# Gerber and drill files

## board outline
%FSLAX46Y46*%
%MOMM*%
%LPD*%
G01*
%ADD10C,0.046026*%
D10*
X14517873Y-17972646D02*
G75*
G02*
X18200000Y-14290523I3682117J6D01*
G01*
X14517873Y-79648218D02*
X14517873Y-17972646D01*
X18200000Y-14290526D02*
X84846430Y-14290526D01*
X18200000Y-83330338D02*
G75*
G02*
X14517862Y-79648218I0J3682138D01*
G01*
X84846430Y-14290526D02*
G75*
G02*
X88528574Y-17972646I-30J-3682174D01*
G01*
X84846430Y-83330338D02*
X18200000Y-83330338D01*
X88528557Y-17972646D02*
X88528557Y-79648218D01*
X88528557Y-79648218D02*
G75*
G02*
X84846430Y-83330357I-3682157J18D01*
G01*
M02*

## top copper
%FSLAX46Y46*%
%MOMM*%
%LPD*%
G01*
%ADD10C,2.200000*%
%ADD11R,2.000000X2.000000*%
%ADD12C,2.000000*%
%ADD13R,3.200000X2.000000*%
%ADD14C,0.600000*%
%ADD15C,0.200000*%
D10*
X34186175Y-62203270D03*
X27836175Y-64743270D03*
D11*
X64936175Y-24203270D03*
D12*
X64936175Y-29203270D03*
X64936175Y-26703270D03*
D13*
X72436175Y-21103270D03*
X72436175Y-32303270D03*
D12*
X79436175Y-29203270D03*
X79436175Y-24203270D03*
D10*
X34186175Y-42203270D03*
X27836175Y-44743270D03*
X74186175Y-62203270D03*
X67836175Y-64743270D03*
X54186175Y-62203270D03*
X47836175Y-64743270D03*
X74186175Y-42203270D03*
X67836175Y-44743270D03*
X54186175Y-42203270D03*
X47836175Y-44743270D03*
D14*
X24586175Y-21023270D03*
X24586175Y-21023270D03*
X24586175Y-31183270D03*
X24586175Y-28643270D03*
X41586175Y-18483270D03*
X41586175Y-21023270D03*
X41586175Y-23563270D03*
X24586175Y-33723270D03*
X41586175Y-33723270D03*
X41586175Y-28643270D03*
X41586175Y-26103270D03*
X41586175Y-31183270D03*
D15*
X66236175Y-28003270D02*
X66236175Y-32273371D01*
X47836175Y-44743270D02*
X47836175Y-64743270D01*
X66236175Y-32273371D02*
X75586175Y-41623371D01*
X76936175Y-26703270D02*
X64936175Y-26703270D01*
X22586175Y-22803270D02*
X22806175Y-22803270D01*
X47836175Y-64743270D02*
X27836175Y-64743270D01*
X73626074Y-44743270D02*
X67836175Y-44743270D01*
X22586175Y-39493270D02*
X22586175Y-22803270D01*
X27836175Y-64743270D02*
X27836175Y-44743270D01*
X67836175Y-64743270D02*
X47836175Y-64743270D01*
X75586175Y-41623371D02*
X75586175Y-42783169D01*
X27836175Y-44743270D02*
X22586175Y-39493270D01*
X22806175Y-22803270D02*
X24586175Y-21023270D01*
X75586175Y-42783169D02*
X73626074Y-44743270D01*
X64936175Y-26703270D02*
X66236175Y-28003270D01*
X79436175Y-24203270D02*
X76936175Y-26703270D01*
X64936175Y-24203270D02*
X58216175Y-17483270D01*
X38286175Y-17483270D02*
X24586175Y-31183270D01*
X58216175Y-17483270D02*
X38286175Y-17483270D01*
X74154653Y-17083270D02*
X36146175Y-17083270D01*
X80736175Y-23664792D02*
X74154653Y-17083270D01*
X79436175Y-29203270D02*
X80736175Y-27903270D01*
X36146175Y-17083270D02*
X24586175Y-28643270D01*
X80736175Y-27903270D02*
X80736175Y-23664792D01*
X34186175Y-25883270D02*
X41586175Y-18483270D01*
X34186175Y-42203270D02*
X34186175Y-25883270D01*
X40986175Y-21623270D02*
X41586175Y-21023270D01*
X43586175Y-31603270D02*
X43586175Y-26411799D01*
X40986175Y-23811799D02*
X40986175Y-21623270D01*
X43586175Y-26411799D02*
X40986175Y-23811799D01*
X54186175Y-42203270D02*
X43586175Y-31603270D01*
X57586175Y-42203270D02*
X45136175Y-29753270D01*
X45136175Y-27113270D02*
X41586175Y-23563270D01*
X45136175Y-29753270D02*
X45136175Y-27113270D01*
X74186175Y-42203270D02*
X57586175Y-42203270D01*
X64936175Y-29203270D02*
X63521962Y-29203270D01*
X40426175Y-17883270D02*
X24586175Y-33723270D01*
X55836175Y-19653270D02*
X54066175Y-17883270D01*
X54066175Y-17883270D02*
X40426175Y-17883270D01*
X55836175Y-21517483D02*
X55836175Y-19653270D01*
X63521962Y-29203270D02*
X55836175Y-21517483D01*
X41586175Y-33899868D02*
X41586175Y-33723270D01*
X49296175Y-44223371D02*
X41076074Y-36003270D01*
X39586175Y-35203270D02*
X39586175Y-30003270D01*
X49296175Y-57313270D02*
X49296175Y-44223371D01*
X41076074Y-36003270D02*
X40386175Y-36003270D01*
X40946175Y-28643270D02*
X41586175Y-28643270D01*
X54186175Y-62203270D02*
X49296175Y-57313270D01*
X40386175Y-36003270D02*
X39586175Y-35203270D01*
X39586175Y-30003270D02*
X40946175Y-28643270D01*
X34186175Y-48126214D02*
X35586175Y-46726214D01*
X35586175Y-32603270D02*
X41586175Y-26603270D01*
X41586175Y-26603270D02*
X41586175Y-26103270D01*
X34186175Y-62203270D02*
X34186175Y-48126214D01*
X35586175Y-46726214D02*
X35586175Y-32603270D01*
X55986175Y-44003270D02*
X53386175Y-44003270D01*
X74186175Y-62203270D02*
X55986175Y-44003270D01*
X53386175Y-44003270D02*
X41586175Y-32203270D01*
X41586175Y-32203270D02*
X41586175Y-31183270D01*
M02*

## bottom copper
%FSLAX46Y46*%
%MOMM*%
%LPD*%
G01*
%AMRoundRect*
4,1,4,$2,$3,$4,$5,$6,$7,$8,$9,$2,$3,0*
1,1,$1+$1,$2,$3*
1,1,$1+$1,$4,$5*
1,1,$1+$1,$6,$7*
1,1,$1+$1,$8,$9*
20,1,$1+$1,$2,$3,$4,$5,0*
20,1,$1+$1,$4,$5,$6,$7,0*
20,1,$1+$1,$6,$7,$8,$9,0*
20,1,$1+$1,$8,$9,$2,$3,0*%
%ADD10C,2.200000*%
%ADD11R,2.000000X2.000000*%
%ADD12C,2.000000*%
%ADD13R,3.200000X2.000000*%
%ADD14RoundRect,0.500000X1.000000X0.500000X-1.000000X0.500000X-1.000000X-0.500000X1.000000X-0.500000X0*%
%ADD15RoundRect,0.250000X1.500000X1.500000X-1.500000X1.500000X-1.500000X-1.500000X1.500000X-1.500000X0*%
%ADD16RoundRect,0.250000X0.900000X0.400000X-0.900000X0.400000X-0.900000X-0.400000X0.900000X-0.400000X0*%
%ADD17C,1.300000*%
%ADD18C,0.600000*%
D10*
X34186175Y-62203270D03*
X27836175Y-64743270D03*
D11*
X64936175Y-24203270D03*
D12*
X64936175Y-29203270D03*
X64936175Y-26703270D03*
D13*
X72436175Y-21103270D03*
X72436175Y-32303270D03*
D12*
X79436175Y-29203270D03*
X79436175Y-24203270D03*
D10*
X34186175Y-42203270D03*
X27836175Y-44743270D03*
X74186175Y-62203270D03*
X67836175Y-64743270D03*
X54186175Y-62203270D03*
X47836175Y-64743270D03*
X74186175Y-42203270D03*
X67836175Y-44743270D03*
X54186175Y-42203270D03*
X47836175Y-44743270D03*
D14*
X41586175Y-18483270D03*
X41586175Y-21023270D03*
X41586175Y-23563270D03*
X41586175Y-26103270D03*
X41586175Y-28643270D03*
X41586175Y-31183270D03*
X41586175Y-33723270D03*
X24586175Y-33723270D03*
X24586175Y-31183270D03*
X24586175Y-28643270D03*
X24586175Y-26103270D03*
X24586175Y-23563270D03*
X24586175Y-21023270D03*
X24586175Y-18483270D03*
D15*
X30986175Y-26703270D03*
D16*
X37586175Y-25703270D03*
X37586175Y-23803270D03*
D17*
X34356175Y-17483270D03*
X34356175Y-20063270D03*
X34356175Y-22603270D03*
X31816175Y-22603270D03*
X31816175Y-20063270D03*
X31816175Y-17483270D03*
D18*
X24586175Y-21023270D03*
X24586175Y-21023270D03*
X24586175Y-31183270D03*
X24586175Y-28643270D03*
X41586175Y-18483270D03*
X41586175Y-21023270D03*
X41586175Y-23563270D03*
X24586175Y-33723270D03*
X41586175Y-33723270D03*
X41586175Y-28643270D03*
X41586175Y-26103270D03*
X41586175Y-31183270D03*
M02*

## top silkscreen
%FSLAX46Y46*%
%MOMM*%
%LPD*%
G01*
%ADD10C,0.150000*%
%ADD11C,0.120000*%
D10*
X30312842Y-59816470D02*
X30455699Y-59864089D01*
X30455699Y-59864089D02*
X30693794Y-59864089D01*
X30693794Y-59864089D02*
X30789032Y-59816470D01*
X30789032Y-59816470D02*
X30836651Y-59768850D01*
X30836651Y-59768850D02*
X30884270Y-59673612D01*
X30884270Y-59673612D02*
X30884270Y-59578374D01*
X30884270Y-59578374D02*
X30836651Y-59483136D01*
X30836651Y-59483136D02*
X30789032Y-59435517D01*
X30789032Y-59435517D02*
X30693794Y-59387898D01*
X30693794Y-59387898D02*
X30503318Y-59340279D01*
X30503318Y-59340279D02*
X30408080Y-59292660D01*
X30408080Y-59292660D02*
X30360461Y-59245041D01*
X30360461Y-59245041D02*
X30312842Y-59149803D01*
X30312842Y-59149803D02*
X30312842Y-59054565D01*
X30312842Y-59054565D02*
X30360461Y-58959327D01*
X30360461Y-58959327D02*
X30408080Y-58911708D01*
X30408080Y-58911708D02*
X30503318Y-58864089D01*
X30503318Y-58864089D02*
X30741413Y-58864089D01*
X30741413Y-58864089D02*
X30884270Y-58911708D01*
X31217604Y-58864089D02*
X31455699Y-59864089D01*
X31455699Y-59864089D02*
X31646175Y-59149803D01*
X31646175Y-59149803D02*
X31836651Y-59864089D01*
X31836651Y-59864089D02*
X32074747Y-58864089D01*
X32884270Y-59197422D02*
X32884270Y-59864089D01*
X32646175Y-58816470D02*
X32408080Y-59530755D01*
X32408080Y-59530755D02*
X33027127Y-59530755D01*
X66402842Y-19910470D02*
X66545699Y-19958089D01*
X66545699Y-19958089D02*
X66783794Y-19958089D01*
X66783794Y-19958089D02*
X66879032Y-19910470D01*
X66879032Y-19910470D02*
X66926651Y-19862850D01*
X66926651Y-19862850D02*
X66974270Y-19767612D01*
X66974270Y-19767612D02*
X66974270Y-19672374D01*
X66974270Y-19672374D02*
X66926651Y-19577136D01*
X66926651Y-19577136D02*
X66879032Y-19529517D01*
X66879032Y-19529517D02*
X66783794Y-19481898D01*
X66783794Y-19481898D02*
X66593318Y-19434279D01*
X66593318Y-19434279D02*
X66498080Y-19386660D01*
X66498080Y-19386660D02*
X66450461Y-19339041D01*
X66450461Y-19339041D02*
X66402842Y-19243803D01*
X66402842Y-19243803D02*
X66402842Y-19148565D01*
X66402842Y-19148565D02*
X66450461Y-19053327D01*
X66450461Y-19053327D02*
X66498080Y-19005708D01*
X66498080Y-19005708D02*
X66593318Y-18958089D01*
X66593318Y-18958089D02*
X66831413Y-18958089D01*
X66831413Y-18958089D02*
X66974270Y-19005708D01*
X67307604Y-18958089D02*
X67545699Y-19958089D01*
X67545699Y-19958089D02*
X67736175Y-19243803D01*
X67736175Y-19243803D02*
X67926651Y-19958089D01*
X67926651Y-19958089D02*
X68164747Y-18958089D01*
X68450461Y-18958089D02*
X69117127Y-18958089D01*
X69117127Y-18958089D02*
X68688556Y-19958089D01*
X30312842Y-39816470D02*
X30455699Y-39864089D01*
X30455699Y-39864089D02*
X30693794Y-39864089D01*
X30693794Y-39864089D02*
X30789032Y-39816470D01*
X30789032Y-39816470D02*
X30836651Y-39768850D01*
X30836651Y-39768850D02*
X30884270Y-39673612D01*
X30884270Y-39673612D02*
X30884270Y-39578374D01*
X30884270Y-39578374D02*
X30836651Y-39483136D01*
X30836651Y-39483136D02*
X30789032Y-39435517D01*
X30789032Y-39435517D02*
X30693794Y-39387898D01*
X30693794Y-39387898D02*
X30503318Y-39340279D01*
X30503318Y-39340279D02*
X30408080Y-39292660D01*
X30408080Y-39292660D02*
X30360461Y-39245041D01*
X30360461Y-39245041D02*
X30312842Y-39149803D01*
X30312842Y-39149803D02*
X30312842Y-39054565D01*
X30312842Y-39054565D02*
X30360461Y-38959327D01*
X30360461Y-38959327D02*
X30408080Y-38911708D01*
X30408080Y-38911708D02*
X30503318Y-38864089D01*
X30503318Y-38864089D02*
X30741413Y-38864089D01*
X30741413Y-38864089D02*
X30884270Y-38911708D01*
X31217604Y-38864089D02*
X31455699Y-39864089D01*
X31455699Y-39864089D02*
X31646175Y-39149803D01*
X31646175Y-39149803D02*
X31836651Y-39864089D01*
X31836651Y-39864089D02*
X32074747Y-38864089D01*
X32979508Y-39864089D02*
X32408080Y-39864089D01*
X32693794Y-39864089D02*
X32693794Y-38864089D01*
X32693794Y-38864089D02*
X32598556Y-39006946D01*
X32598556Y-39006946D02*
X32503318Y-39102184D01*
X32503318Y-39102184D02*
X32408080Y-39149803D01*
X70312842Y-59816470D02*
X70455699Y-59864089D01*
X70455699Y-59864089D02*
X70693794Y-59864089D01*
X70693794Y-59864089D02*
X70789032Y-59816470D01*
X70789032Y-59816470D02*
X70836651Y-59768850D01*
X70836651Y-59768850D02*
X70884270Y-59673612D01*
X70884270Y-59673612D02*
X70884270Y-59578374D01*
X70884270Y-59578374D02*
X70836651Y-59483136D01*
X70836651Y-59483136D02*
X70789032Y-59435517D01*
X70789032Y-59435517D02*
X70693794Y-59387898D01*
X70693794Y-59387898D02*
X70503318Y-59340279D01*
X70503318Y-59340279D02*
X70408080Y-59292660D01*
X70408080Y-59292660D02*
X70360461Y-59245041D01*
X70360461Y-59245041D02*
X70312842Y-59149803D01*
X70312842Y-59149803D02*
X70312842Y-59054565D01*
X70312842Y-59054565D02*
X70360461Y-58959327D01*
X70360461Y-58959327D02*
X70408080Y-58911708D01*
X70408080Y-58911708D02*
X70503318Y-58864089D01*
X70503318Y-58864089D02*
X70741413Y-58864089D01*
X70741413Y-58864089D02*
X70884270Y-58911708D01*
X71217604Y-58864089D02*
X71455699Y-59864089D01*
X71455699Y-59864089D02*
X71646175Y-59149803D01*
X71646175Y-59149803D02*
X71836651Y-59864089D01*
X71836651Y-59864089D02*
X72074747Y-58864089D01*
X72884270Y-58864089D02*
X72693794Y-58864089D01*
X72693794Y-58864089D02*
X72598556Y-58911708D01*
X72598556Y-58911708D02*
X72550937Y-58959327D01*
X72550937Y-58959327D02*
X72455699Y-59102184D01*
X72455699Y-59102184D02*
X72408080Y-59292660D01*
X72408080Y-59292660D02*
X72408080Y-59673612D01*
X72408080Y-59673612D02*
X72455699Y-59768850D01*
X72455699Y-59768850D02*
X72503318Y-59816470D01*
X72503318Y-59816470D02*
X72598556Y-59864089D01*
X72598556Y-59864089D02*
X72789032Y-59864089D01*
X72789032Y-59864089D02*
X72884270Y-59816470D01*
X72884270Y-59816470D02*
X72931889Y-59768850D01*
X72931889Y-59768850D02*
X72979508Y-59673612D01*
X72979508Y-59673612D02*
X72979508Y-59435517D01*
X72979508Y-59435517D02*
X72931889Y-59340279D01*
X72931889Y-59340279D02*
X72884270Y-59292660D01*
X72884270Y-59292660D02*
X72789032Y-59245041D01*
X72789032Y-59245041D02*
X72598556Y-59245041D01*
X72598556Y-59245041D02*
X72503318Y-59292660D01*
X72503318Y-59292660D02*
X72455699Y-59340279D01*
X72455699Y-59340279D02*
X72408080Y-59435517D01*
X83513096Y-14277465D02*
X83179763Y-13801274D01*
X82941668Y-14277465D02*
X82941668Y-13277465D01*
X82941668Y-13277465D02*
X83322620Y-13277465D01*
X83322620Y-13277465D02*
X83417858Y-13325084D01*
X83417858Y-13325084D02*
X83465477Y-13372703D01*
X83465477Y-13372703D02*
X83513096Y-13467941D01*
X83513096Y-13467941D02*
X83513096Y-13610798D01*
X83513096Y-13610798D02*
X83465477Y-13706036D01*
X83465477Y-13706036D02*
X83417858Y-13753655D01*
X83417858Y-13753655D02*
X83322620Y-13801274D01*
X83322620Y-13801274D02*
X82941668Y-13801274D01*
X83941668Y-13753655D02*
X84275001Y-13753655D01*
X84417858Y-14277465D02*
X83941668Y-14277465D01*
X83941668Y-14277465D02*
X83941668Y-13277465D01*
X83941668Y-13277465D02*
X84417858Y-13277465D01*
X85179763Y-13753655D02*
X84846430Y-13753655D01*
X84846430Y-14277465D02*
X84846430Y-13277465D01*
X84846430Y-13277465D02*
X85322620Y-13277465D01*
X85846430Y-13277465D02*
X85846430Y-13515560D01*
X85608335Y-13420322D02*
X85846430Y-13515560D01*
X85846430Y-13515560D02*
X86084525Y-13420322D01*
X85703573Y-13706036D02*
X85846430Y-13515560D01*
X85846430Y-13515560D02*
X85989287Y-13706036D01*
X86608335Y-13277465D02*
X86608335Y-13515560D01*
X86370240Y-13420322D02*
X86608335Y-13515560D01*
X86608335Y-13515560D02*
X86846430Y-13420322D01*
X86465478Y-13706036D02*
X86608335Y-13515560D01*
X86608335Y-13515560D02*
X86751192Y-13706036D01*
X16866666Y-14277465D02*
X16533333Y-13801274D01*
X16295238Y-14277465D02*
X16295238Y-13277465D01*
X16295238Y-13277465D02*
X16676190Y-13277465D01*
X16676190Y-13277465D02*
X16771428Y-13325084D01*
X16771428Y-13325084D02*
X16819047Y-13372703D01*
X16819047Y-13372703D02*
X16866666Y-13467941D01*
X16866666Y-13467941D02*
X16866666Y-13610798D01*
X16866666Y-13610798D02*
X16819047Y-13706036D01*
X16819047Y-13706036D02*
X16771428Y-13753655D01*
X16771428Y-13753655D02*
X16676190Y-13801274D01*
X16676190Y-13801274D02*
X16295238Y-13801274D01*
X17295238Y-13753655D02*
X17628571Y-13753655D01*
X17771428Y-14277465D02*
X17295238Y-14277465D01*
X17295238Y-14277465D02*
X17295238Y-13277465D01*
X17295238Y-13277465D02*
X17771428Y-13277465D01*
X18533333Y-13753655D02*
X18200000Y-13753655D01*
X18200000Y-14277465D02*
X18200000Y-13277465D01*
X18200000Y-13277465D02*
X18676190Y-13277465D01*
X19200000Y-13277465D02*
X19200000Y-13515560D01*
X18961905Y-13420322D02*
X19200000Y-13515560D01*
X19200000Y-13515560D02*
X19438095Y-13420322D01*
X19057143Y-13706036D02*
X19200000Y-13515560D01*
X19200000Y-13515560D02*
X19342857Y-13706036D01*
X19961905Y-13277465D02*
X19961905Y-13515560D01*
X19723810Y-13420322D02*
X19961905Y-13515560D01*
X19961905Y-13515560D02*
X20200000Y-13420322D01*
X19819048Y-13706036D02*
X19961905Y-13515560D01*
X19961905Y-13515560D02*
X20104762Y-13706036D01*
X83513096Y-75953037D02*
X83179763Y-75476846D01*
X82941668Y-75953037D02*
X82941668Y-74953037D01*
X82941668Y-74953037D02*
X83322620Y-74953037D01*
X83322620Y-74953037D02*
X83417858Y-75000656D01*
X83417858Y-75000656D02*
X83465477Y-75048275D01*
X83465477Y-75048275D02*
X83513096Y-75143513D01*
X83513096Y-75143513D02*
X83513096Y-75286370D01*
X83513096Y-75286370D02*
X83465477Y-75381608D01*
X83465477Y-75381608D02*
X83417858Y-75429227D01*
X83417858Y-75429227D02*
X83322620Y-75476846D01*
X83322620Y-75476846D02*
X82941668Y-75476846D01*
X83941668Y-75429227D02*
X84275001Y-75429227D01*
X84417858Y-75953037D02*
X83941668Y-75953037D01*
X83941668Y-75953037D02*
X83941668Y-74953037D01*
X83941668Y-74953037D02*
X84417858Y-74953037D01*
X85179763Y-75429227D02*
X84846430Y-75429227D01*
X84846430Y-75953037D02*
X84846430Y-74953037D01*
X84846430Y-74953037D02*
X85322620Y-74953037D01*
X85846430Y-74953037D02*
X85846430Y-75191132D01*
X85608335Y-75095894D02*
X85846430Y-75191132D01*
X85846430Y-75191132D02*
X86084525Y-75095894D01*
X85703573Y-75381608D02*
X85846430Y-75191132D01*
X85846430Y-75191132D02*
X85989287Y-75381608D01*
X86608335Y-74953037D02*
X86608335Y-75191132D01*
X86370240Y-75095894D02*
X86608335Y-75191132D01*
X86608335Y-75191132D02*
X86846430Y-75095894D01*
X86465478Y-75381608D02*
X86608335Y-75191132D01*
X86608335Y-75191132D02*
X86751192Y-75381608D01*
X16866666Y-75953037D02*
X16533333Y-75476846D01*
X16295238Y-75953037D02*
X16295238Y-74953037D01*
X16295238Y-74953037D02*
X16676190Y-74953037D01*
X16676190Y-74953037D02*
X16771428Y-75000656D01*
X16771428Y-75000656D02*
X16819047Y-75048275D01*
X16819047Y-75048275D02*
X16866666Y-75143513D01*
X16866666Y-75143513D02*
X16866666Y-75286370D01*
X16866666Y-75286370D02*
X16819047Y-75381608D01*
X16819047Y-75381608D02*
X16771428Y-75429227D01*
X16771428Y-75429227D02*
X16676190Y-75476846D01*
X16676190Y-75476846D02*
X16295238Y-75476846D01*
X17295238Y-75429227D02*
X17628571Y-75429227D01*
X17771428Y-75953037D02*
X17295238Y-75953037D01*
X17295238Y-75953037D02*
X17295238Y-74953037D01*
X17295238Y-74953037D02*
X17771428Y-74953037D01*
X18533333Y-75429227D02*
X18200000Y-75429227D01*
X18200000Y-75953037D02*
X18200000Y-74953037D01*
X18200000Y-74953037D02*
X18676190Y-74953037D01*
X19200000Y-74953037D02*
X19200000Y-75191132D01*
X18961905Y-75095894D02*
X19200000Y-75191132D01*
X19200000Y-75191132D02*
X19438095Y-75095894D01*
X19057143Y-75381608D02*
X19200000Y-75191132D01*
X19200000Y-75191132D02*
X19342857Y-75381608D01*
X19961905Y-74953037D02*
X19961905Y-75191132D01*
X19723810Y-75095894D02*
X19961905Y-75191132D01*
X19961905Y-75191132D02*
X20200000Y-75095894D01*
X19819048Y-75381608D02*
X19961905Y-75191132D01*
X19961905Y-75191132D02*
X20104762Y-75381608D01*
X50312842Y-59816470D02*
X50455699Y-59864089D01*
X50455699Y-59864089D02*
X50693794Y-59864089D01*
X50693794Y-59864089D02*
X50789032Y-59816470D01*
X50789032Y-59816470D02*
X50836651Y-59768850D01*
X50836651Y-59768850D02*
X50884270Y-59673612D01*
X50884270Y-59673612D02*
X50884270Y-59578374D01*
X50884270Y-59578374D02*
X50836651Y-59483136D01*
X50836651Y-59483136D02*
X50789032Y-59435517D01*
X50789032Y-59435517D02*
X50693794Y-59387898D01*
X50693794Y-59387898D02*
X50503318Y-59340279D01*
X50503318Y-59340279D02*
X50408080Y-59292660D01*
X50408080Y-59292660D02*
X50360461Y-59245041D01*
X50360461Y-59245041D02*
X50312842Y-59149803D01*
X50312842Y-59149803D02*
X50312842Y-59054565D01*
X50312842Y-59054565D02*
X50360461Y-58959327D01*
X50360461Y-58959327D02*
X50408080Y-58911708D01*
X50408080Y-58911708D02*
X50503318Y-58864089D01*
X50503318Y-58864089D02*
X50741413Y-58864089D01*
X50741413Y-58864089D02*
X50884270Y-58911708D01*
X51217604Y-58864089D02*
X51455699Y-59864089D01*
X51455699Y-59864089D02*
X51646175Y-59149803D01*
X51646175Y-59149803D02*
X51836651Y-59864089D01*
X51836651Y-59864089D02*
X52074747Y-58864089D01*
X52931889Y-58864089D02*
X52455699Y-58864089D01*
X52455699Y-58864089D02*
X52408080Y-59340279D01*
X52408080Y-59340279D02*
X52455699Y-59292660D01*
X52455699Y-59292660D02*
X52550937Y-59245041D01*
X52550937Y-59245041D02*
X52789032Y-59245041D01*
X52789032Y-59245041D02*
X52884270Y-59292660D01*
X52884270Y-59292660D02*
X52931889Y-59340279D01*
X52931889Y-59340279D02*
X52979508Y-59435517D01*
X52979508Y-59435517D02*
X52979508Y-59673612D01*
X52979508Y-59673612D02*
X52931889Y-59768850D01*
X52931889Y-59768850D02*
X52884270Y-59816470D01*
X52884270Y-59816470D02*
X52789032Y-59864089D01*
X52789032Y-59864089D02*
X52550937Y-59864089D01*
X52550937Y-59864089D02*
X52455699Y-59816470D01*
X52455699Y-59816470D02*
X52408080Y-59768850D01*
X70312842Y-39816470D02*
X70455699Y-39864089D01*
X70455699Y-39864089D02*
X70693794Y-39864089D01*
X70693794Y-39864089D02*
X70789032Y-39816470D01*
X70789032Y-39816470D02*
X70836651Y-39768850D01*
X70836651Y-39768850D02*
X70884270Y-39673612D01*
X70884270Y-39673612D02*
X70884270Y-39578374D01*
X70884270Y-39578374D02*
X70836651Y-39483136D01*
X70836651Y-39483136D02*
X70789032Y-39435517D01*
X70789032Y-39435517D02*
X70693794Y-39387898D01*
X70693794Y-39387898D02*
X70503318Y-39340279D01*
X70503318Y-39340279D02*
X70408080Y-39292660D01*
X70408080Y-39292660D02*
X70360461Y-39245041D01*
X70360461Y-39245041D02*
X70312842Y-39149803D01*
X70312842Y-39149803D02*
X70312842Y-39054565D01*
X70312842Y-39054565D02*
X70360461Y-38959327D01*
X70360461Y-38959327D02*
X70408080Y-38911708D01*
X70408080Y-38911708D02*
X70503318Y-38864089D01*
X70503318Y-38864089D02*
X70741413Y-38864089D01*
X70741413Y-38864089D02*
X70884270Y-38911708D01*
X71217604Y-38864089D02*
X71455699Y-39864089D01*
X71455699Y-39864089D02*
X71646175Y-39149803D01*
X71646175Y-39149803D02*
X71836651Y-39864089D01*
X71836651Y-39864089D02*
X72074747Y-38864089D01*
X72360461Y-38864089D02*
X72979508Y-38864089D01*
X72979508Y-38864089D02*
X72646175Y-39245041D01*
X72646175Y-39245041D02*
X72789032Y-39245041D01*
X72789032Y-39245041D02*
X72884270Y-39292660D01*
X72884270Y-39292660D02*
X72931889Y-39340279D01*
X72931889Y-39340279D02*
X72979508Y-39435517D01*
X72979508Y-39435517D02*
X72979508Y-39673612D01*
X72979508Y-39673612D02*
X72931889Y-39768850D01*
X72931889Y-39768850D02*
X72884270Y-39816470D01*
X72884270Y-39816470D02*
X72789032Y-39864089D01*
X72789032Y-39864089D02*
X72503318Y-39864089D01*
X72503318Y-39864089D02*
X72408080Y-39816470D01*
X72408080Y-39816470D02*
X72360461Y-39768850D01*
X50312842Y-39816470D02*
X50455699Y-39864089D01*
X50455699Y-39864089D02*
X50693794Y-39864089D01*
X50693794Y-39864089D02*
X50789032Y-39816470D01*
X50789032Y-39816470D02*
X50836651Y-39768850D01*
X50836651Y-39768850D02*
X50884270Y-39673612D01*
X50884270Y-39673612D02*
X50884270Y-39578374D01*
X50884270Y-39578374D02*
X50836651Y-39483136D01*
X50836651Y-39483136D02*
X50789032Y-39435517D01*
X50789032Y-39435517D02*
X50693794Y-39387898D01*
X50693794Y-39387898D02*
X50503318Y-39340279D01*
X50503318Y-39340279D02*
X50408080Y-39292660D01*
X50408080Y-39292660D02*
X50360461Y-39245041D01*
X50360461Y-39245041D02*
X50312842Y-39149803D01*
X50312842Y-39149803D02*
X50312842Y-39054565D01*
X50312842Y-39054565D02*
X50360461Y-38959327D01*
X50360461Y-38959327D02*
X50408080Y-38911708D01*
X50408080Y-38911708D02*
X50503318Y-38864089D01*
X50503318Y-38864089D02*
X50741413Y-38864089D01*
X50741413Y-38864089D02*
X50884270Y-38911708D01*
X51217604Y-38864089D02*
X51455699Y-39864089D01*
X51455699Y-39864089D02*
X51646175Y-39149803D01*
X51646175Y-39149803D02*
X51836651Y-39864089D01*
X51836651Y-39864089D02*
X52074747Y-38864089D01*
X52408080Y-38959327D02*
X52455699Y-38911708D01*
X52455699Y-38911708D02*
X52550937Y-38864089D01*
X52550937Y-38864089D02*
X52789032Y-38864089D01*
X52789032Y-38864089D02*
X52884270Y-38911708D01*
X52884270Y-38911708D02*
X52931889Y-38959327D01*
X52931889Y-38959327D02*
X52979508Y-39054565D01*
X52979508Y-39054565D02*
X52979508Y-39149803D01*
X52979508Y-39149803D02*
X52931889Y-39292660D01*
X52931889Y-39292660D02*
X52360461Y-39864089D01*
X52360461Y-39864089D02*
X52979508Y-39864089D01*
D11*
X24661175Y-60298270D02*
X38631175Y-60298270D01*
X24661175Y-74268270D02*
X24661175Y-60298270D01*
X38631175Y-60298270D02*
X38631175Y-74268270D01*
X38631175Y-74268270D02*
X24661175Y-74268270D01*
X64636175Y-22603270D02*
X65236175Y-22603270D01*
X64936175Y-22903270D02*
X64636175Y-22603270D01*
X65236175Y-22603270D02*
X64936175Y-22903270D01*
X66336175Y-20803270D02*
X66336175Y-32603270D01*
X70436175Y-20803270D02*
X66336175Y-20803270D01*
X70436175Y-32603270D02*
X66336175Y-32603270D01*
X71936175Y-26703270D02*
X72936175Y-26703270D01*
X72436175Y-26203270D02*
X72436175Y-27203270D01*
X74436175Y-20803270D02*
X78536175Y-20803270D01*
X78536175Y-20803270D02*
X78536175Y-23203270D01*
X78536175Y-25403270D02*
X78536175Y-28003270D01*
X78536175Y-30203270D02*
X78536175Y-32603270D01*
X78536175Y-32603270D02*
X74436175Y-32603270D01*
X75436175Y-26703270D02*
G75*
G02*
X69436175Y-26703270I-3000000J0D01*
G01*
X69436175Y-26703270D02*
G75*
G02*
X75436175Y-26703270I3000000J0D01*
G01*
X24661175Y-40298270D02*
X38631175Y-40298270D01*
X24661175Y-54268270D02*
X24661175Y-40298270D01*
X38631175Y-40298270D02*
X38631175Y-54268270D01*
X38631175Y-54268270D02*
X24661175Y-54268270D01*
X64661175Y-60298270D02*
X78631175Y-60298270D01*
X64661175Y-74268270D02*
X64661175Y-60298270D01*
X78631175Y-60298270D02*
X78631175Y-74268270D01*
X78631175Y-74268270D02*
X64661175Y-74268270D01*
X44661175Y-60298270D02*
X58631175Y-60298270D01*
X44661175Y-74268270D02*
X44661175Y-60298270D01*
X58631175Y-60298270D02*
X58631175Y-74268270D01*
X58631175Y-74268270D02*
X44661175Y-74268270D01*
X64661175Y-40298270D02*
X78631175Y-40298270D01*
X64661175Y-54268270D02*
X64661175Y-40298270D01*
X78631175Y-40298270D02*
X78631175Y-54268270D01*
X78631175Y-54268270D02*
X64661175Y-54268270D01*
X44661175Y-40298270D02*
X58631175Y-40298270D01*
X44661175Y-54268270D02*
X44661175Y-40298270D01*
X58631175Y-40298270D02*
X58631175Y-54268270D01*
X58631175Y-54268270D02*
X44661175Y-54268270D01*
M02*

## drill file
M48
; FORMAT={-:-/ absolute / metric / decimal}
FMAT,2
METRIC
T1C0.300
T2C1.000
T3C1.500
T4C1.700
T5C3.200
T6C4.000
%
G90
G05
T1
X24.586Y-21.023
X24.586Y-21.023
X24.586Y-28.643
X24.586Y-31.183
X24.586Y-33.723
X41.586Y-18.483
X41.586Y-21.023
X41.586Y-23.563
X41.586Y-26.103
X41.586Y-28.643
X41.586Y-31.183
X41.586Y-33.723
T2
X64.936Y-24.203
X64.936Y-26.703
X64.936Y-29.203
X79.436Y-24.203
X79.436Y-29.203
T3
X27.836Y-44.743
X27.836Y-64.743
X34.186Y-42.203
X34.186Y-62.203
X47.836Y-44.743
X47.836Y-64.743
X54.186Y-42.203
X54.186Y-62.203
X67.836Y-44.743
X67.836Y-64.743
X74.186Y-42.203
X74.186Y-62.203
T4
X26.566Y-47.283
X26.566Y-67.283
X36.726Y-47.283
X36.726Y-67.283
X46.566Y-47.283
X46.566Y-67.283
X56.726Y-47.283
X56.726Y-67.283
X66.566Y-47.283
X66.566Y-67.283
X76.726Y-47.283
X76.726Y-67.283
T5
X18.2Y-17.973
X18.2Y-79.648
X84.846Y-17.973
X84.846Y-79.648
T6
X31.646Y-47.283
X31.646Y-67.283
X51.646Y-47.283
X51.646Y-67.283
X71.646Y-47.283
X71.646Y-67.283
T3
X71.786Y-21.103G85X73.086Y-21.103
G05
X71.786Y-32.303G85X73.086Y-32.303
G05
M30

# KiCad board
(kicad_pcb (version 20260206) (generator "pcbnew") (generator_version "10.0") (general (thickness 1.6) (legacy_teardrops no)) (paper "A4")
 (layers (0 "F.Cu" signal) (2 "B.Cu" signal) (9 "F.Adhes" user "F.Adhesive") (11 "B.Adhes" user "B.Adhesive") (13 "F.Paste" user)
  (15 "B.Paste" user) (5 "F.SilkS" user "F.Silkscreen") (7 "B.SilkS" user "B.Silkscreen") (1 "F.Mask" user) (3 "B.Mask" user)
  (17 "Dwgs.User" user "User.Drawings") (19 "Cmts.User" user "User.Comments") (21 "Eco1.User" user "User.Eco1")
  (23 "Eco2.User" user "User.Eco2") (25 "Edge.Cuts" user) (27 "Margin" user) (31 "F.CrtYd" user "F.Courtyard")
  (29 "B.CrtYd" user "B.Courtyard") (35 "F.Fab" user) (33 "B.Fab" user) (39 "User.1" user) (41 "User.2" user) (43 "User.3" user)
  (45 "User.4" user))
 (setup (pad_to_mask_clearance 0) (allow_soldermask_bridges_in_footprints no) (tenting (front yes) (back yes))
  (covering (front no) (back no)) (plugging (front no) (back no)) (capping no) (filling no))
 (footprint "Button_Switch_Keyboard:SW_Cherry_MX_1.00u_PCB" (layer "F.Cu") (at 34.186175 62.20327)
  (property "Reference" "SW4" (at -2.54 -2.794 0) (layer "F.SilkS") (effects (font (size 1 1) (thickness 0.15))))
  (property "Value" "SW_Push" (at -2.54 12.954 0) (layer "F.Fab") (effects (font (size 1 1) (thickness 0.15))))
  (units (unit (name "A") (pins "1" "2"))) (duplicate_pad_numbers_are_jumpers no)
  (fp_line (start -9.525 -1.905) (end 4.445 -1.905) (stroke (width 0.12) (type solid)) (layer "F.SilkS"))
  (fp_line (start -9.525 12.065) (end -9.525 -1.905) (stroke (width 0.12) (type solid)) (layer "F.SilkS"))
  (fp_line (start 4.445 -1.905) (end 4.445 12.065) (stroke (width 0.12) (type solid)) (layer "F.SilkS"))
  (fp_line (start 4.445 12.065) (end -9.525 12.065) (stroke (width 0.12) (type solid)) (layer "F.SilkS"))
  (pad "" np_thru_hole circle (at -7.62 5.08) (size 1.7 1.7) (drill 1.7) (layers "*.Cu" "*.Mask"))
  (pad "" np_thru_hole circle (at -2.54 5.08) (size 4 4) (drill 4) (layers "*.Cu" "*.Mask"))
  (pad "" np_thru_hole circle (at 2.54 5.08) (size 1.7 1.7) (drill 1.7) (layers "*.Cu" "*.Mask"))
  (pad "1" thru_hole circle (at 0 0) (size 2.2 2.2) (drill 1.5) (layers "*.Cu" "*.Mask") (remove_unused_layers no)
   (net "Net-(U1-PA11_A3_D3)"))
  (pad "2" thru_hole circle (at -6.35 2.54) (size 2.2 2.2) (drill 1.5) (layers "*.Cu" "*.Mask") (remove_unused_layers no)
   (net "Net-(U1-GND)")))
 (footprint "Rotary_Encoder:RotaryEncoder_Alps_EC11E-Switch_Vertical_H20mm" (layer "F.Cu") (at 64.936175 24.20327)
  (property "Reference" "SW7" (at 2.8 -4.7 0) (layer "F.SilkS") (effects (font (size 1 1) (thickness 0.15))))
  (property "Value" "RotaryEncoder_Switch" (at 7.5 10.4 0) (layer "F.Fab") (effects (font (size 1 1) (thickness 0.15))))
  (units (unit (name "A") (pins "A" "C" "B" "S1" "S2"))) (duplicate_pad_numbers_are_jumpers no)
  (fp_line (start -0.3 -1.6) (end 0.3 -1.6) (stroke (width 0.12) (type solid)) (layer "F.SilkS"))
  (fp_line (start 0 -1.3) (end -0.3 -1.6) (stroke (width 0.12) (type solid)) (layer "F.SilkS"))
  (fp_line (start 0.3 -1.6) (end 0 -1.3) (stroke (width 0.12) (type solid)) (layer "F.SilkS"))
  (fp_line (start 1.4 -3.4) (end 1.4 8.4) (stroke (width 0.12) (type solid)) (layer "F.SilkS"))
  (fp_line (start 5.5 -3.4) (end 1.4 -3.4) (stroke (width 0.12) (type solid)) (layer "F.SilkS"))
  (fp_line (start 5.5 8.4) (end 1.4 8.4) (stroke (width 0.12) (type solid)) (layer "F.SilkS"))
  (fp_line (start 7 2.5) (end 8 2.5) (stroke (width 0.12) (type solid)) (layer "F.SilkS"))
  (fp_line (start 7.5 2) (end 7.5 3) (stroke (width 0.12) (type solid)) (layer "F.SilkS"))
  (fp_line (start 9.5 -3.4) (end 13.6 -3.4) (stroke (width 0.12) (type solid)) (layer "F.SilkS"))
  (fp_line (start 13.6 -3.4) (end 13.6 -1) (stroke (width 0.12) (type solid)) (layer "F.SilkS"))
  (fp_line (start 13.6 1.2) (end 13.6 3.8) (stroke (width 0.12) (type solid)) (layer "F.SilkS"))
  (fp_line (start 13.6 6) (end 13.6 8.4) (stroke (width 0.12) (type solid)) (layer "F.SilkS"))
  (fp_line (start 13.6 8.4) (end 9.5 8.4) (stroke (width 0.12) (type solid)) (layer "F.SilkS"))
  (fp_circle (center 7.5 2.5) (end 10.5 2.5) (stroke (width 0.12) (type solid)) (fill no) (layer "F.SilkS"))
  (pad "A" thru_hole rect (at 0 0) (size 2 2) (drill 1) (layers "*.Cu" "*.Mask") (remove_unused_layers no) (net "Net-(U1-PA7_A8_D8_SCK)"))
  (pad "B" thru_hole circle (at 0 5) (size 2 2) (drill 1) (layers "*.Cu" "*.Mask") (remove_unused_layers no) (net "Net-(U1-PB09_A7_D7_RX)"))
  (pad "C" thru_hole circle (at 0 2.5) (size 2 2) (drill 1) (layers "*.Cu" "*.Mask") (remove_unused_layers no) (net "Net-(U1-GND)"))
  (pad "MP" thru_hole rect (at 7.5 -3.1) (size 3.2 2) (drill oval 2.8 1.5) (layers "*.Cu" "*.Mask") (remove_unused_layers no))
  (pad "MP" thru_hole rect (at 7.5 8.1) (size 3.2 2) (drill oval 2.8 1.5) (layers "*.Cu" "*.Mask") (remove_unused_layers no))
  (pad "S1" thru_hole circle (at 14.5 5) (size 2 2) (drill 1) (layers "*.Cu" "*.Mask") (remove_unused_layers no)
   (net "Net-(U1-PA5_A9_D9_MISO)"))
  (pad "S2" thru_hole circle (at 14.5 0) (size 2 2) (drill 1) (layers "*.Cu" "*.Mask") (remove_unused_layers no) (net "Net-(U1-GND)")))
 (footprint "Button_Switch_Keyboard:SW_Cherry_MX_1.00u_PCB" (layer "F.Cu") (at 34.186175 42.20327)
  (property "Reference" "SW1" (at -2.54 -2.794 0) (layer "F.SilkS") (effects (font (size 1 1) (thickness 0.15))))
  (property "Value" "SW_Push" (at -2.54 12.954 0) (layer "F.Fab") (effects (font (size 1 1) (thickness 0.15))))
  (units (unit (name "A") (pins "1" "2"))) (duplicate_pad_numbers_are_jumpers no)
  (fp_line (start -9.525 -1.905) (end 4.445 -1.905) (stroke (width 0.12) (type solid)) (layer "F.SilkS"))
  (fp_line (start -9.525 12.065) (end -9.525 -1.905) (stroke (width 0.12) (type solid)) (layer "F.SilkS"))
  (fp_line (start 4.445 -1.905) (end 4.445 12.065) (stroke (width 0.12) (type solid)) (layer "F.SilkS"))
  (fp_line (start 4.445 12.065) (end -9.525 12.065) (stroke (width 0.12) (type solid)) (layer "F.SilkS"))
  (pad "" np_thru_hole circle (at -7.62 5.08) (size 1.7 1.7) (drill 1.7) (layers "*.Cu" "*.Mask"))
  (pad "" np_thru_hole circle (at -2.54 5.08) (size 4 4) (drill 4) (layers "*.Cu" "*.Mask"))
  (pad "" np_thru_hole circle (at 2.54 5.08) (size 1.7 1.7) (drill 1.7) (layers "*.Cu" "*.Mask"))
  (pad "1" thru_hole circle (at 0 0) (size 2.2 2.2) (drill 1.5) (layers "*.Cu" "*.Mask") (remove_unused_layers no)
   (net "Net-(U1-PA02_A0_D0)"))
  (pad "2" thru_hole circle (at -6.35 2.54) (size 2.2 2.2) (drill 1.5) (layers "*.Cu" "*.Mask") (remove_unused_layers no)
   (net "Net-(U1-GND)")))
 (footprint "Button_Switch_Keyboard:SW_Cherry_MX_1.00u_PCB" (layer "F.Cu") (at 74.186175 62.20327)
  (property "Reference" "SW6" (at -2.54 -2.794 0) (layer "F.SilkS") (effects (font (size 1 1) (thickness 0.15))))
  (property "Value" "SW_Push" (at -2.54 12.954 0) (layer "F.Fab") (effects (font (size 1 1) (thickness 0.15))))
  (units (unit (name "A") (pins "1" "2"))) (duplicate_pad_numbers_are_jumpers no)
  (fp_line (start -9.525 -1.905) (end 4.445 -1.905) (stroke (width 0.12) (type solid)) (layer "F.SilkS"))
  (fp_line (start -9.525 12.065) (end -9.525 -1.905) (stroke (width 0.12) (type solid)) (layer "F.SilkS"))
  (fp_line (start 4.445 -1.905) (end 4.445 12.065) (stroke (width 0.12) (type solid)) (layer "F.SilkS"))
  (fp_line (start 4.445 12.065) (end -9.525 12.065) (stroke (width 0.12) (type solid)) (layer "F.SilkS"))
  (pad "" np_thru_hole circle (at -7.62 5.08) (size 1.7 1.7) (drill 1.7) (layers "*.Cu" "*.Mask"))
  (pad "" np_thru_hole circle (at -2.54 5.08) (size 4 4) (drill 4) (layers "*.Cu" "*.Mask"))
  (pad "" np_thru_hole circle (at 2.54 5.08) (size 1.7 1.7) (drill 1.7) (layers "*.Cu" "*.Mask"))
  (pad "1" thru_hole circle (at 0 0) (size 2.2 2.2) (drill 1.5) (layers "*.Cu" "*.Mask") (remove_unused_layers no)
   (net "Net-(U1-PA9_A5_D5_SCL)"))
  (pad "2" thru_hole circle (at -6.35 2.54) (size 2.2 2.2) (drill 1.5) (layers "*.Cu" "*.Mask") (remove_unused_layers no)
   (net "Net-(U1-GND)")))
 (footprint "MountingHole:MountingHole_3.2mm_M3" (layer "F.Cu") (at 84.84643 17.972646)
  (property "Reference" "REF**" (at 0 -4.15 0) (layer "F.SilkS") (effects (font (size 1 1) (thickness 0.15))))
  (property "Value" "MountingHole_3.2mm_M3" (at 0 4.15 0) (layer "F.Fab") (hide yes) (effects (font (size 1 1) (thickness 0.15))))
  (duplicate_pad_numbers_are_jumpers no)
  (pad "" np_thru_hole circle (at 0 0) (size 3.2 3.2) (drill 3.2) (layers "*.Cu" "*.Mask")))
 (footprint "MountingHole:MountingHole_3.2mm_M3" (layer "F.Cu") (at 18.2 17.972646)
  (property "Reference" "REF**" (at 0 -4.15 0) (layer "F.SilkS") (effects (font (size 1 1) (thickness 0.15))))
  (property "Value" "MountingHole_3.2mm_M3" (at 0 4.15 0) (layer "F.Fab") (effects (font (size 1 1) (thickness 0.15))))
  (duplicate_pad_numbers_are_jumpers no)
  (pad "" np_thru_hole circle (at 0 0) (size 3.2 3.2) (drill 3.2) (layers "*.Cu" "*.Mask")))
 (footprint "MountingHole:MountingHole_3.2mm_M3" (layer "F.Cu") (at 84.84643 79.648218)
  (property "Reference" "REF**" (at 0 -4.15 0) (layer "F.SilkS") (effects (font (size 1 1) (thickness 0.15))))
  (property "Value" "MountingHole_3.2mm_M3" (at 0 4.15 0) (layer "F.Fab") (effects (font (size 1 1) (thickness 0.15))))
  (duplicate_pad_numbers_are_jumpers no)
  (pad "" np_thru_hole circle (at 0 0) (size 3.2 3.2) (drill 3.2) (layers "*.Cu" "*.Mask")))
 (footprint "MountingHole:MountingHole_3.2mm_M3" (layer "F.Cu") (at 18.2 79.648218)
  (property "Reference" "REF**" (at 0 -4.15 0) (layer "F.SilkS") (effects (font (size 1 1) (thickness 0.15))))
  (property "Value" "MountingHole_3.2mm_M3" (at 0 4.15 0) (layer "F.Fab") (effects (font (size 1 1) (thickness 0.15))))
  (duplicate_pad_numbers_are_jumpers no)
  (pad "" np_thru_hole circle (at 0 0) (size 3.2 3.2) (drill 3.2) (layers "*.Cu" "*.Mask")))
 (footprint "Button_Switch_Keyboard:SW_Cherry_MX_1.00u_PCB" (layer "F.Cu") (at 54.186175 62.20327)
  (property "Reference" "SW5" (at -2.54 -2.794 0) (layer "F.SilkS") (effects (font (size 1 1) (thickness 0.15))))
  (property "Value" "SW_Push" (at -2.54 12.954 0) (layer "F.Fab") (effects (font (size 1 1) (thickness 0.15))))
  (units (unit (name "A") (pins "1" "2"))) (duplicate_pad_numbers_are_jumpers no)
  (fp_line (start -9.525 -1.905) (end 4.445 -1.905) (stroke (width 0.12) (type solid)) (layer "F.SilkS"))
  (fp_line (start -9.525 12.065) (end -9.525 -1.905) (stroke (width 0.12) (type solid)) (layer "F.SilkS"))
  (fp_line (start 4.445 -1.905) (end 4.445 12.065) (stroke (width 0.12) (type solid)) (layer "F.SilkS"))
  (fp_line (start 4.445 12.065) (end -9.525 12.065) (stroke (width 0.12) (type solid)) (layer "F.SilkS"))
  (pad "" np_thru_hole circle (at -7.62 5.08) (size 1.7 1.7) (drill 1.7) (layers "*.Cu" "*.Mask"))
  (pad "" np_thru_hole circle (at -2.54 5.08) (size 4 4) (drill 4) (layers "*.Cu" "*.Mask"))
  (pad "" np_thru_hole circle (at 2.54 5.08) (size 1.7 1.7) (drill 1.7) (layers "*.Cu" "*.Mask"))
  (pad "1" thru_hole circle (at 0 0) (size 2.2 2.2) (drill 1.5) (layers "*.Cu" "*.Mask") (remove_unused_layers no)
   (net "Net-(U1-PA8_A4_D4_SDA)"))
  (pad "2" thru_hole circle (at -6.35 2.54) (size 2.2 2.2) (drill 1.5) (layers "*.Cu" "*.Mask") (remove_unused_layers no)
   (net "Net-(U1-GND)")))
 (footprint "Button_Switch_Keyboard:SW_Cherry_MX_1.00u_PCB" (layer "F.Cu") (at 74.186175 42.20327)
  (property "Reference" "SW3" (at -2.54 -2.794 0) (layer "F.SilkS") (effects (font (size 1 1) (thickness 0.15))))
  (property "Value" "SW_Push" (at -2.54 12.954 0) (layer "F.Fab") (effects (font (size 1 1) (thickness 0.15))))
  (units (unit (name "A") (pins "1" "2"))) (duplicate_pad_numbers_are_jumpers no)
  (fp_line (start -9.525 -1.905) (end 4.445 -1.905) (stroke (width 0.12) (type solid)) (layer "F.SilkS"))
  (fp_line (start -9.525 12.065) (end -9.525 -1.905) (stroke (width 0.12) (type solid)) (layer "F.SilkS"))
  (fp_line (start 4.445 -1.905) (end 4.445 12.065) (stroke (width 0.12) (type solid)) (layer "F.SilkS"))
  (fp_line (start 4.445 12.065) (end -9.525 12.065) (stroke (width 0.12) (type solid)) (layer "F.SilkS"))
  (pad "" np_thru_hole circle (at -7.62 5.08) (size 1.7 1.7) (drill 1.7) (layers "*.Cu" "*.Mask"))
  (pad "" np_thru_hole circle (at -2.54 5.08) (size 4 4) (drill 4) (layers "*.Cu" "*.Mask"))
  (pad "" np_thru_hole circle (at 2.54 5.08) (size 1.7 1.7) (drill 1.7) (layers "*.Cu" "*.Mask"))
  (pad "1" thru_hole circle (at 0 0) (size 2.2 2.2) (drill 1.5) (layers "*.Cu" "*.Mask") (remove_unused_layers no)
   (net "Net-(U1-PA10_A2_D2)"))
  (pad "2" thru_hole circle (at -6.35 2.54) (size 2.2 2.2) (drill 1.5) (layers "*.Cu" "*.Mask") (remove_unused_layers no)
   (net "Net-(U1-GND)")))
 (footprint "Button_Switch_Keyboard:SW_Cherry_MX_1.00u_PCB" (layer "F.Cu") (at 54.186175 42.20327)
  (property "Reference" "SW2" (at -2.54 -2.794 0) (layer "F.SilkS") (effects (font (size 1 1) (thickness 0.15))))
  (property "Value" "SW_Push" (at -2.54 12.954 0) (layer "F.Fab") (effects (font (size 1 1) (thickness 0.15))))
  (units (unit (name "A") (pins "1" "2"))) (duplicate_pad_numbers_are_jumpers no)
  (fp_line (start -9.525 -1.905) (end 4.445 -1.905) (stroke (width 0.12) (type solid)) (layer "F.SilkS"))
  (fp_line (start -9.525 12.065) (end -9.525 -1.905) (stroke (width 0.12) (type solid)) (layer "F.SilkS"))
  (fp_line (start 4.445 -1.905) (end 4.445 12.065) (stroke (width 0.12) (type solid)) (layer "F.SilkS"))
  (fp_line (start 4.445 12.065) (end -9.525 12.065) (stroke (width 0.12) (type solid)) (layer "F.SilkS"))
  (pad "" np_thru_hole circle (at -7.62 5.08) (size 1.7 1.7) (drill 1.7) (layers "*.Cu" "*.Mask"))
  (pad "" np_thru_hole circle (at -2.54 5.08) (size 4 4) (drill 4) (layers "*.Cu" "*.Mask"))
  (pad "" np_thru_hole circle (at 2.54 5.08) (size 1.7 1.7) (drill 1.7) (layers "*.Cu" "*.Mask"))
  (pad "1" thru_hole circle (at 0 0) (size 2.2 2.2) (drill 1.5) (layers "*.Cu" "*.Mask") (remove_unused_layers no)
   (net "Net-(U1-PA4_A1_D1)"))
  (pad "2" thru_hole circle (at -6.35 2.54) (size 2.2 2.2) (drill 1.5) (layers "*.Cu" "*.Mask") (remove_unused_layers no)
   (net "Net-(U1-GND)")))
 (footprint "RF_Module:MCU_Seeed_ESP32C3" (layer "B.Cu") (at 33.086175 26.10327 180)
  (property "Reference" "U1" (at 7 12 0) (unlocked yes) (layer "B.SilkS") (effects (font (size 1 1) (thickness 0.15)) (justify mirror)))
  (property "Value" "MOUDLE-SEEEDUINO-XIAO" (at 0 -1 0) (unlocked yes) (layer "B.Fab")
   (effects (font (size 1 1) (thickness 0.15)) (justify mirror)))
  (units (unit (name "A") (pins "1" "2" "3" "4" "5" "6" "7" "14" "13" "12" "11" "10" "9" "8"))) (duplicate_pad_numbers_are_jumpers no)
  (pad "" smd roundrect (at 1.1 -1.6 180) (size 1.5 1.5) (layers "B.Paste") (roundrect_rratio 0.1666666667))
  (pad "" smd roundrect (at 1.1 0.4 180) (size 1.5 1.5) (layers "B.Paste") (roundrect_rratio 0.1666666667))
  (pad "" smd roundrect (at 3.1 -1.6 180) (size 1.5 1.5) (layers "B.Paste") (roundrect_rratio 0.1666666667))
  (pad "" smd roundrect (at 3.1 0.4 180) (size 1.5 1.5) (layers "B.Paste") (roundrect_rratio 0.1666666667))
  (pad "1" smd roundrect (at -8.5 7.62 180) (size 3 2) (layers "B.Cu" "B.Mask" "B.Paste") (roundrect_rratio 0.25)
   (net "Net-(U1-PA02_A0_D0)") (thermal_bridge_angle 45))
  (pad "2" smd roundrect (at -8.5 5.08 180) (size 3 2) (layers "B.Cu" "B.Mask" "B.Paste") (roundrect_rratio 0.25) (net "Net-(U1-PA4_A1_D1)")
   (thermal_bridge_angle 45))
  (pad "3" smd roundrect (at -8.5 2.54 180) (size 3 2) (layers "B.Cu" "B.Mask" "B.Paste") (roundrect_rratio 0.25)
   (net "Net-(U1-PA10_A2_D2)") (thermal_bridge_angle 45))
  (pad "4" smd roundrect (at -8.5 0 180) (size 3 2) (layers "B.Cu" "B.Mask" "B.Paste") (roundrect_rratio 0.25) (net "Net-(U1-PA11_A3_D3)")
   (thermal_bridge_angle 45))
  (pad "5" smd roundrect (at -8.5 -2.54 180) (size 3 2) (layers "B.Cu" "B.Mask" "B.Paste") (roundrect_rratio 0.25)
   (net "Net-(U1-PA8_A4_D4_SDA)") (thermal_bridge_angle 45))
  (pad "6" smd roundrect (at -8.5 -5.08 180) (size 3 2) (layers "B.Cu" "B.Mask" "B.Paste") (roundrect_rratio 0.25)
   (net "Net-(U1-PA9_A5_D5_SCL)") (thermal_bridge_angle 45))
  (pad "7" smd roundrect (at -8.5 -7.62 180) (size 3 2) (layers "B.Cu" "B.Mask" "B.Paste") (roundrect_rratio 0.25)
   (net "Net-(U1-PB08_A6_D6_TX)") (thermal_bridge_angle 45))
  (pad "8" smd roundrect (at 8.5 -7.62 180) (size 3 2) (layers "B.Cu" "B.Mask" "B.Paste") (roundrect_rratio 0.25)
   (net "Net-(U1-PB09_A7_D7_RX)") (thermal_bridge_angle 45))
  (pad "9" smd roundrect (at 8.5 -5.08 180) (size 3 2) (layers "B.Cu" "B.Mask" "B.Paste") (roundrect_rratio 0.25)
   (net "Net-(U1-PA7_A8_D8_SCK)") (thermal_bridge_angle 45))
  (pad "10" smd roundrect (at 8.5 -2.54 180) (size 3 2) (layers "B.Cu" "B.Mask" "B.Paste") (roundrect_rratio 0.25)
   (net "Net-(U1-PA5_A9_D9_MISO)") (thermal_bridge_angle 45))
  (pad "11" smd roundrect (at 8.5 0 180) (size 3 2) (layers "B.Cu" "B.Mask" "B.Paste") (roundrect_rratio 0.25)
   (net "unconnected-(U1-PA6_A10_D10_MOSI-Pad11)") (thermal_bridge_angle 45))
  (pad "12" smd roundrect (at 8.5 2.54 180) (size 3 2) (layers "B.Cu" "B.Mask" "B.Paste") (roundrect_rratio 0.25)
   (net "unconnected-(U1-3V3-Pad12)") (thermal_bridge_angle 45))
  (pad "13" smd roundrect (at 8.5 5.08 180) (size 3 2) (layers "B.Cu" "B.Mask" "B.Paste") (roundrect_rratio 0.25) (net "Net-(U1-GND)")
   (thermal_bridge_angle 45))
  (pad "14" smd roundrect (at 8.5 7.62 180) (size 3 2) (layers "B.Cu" "B.Mask" "B.Paste") (roundrect_rratio 0.25)
   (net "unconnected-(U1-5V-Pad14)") (thermal_bridge_angle 45))
  (pad "15" smd roundrect (at 2.1 -0.6 180) (size 3.5 3.5) (layers "B.Cu" "B.Mask") (roundrect_rratio 0.07142857143))
  (pad "16" smd roundrect (at -4.5 0.4 180) (size 2.3 1.3) (layers "B.Cu" "B.Mask" "B.Paste") (roundrect_rratio 0.1923076923))
  (pad "17" smd roundrect (at -4.5 2.3 180) (size 2.3 1.3) (layers "B.Cu" "B.Mask" "B.Paste") (roundrect_rratio 0.1923076923))
  (pad "18" smd circle (at -1.27 8.62 180) (size 1.3 1.3) (layers "B.Cu" "B.Mask" "B.Paste"))
  (pad "19" smd circle (at -1.27 6.04 180) (size 1.3 1.3) (layers "B.Cu" "B.Mask" "B.Paste"))
  (pad "20" smd circle (at -1.27 3.5 180) (size 1.3 1.3) (layers "B.Cu" "B.Mask" "B.Paste"))
  (pad "21" smd circle (at 1.27 3.5 180) (size 1.3 1.3) (layers "B.Cu" "B.Mask" "B.Paste"))
  (pad "22" smd circle (at 1.27 6.04 180) (size 1.3 1.3) (layers "B.Cu" "B.Mask" "B.Paste"))
  (pad "23" smd circle (at 1.27 8.62 180) (size 1.3 1.3) (layers "B.Cu" "B.Mask" "B.Paste")))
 (gr_arc (start 14.517873 17.972646) (mid 15.596343 15.368989) (end 18.2 14.290526) (stroke (width 0.046026) (type default))
  (layer "Edge.Cuts"))
 (gr_line (start 14.517873 79.648218) (end 14.517873 17.972646) (stroke (width 0.046026) (type default)) (layer "Edge.Cuts"))
 (gr_line (start 18.2 14.290526) (end 84.84643 14.290526) (stroke (width 0.046026) (type default)) (layer "Edge.Cuts"))
 (gr_arc (start 18.2 83.330338) (mid 15.596348 82.25187) (end 14.517873 79.648218) (stroke (width 0.046026) (type default))
  (layer "Edge.Cuts"))
 (gr_arc (start 84.84643 14.290526) (mid 87.450082 15.368994) (end 88.528557 17.972646) (stroke (width 0.046026) (type default))
  (layer "Edge.Cuts"))
 (gr_line (start 84.84643 83.330338) (end 18.2 83.330338) (stroke (width 0.046026) (type default)) (layer "Edge.Cuts"))
 (gr_line (start 88.528557 17.972646) (end 88.528557 79.648218) (stroke (width 0.046026) (type default)) (layer "Edge.Cuts"))
 (gr_arc (start 88.528557 79.648218) (mid 87.450087 82.251875) (end 84.84643 83.330338) (stroke (width 0.046026) (type default))
  (layer "Edge.Cuts"))
 (segment (start 66.236175 28.00327) (end 66.236175 32.273371) (width 0.2) (layer "F.Cu") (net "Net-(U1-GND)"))
 (segment (start 47.836175 44.74327) (end 47.836175 64.74327) (width 0.2) (layer "F.Cu") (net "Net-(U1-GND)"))
 (segment (start 66.236175 32.273371) (end 75.586175 41.623371) (width 0.2) (layer "F.Cu") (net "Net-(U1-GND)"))
 (segment (start 76.936175 26.70327) (end 64.936175 26.70327) (width 0.2) (layer "F.Cu") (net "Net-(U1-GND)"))
 (segment (start 22.586175 22.80327) (end 22.806175 22.80327) (width 0.2) (layer "F.Cu") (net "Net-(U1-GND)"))
 (segment (start 47.836175 64.74327) (end 27.836175 64.74327) (width 0.2) (layer "F.Cu") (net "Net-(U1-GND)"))
 (segment (start 73.626074 44.74327) (end 67.836175 44.74327) (width 0.2) (layer "F.Cu") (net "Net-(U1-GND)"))
 (segment (start 22.586175 39.49327) (end 22.586175 22.80327) (width 0.2) (layer "F.Cu") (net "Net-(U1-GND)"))
 (segment (start 27.836175 64.74327) (end 27.836175 44.74327) (width 0.2) (layer "F.Cu") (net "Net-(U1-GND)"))
 (segment (start 67.836175 64.74327) (end 47.836175 64.74327) (width 0.2) (layer "F.Cu") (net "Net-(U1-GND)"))
 (segment (start 75.586175 41.623371) (end 75.586175 42.783169) (width 0.2) (layer "F.Cu") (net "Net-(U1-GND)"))
 (segment (start 27.836175 44.74327) (end 22.586175 39.49327) (width 0.2) (layer "F.Cu") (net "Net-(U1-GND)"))
 (segment (start 22.806175 22.80327) (end 24.586175 21.02327) (width 0.2) (layer "F.Cu") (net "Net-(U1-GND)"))
 (segment (start 75.586175 42.783169) (end 73.626074 44.74327) (width 0.2) (layer "F.Cu") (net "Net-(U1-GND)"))
 (segment (start 64.936175 26.70327) (end 66.236175 28.00327) (width 0.2) (layer "F.Cu") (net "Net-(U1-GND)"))
 (segment (start 79.436175 24.20327) (end 76.936175 26.70327) (width 0.2) (layer "F.Cu") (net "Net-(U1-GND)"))
 (via (at 24.586175 21.02327) (size 0.6) (drill 0.3) (layers "F.Cu" "B.Cu") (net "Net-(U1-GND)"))
 (via (at 24.586175 21.02327) (size 0.6) (drill 0.3) (layers "F.Cu" "B.Cu") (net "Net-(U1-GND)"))
 (segment (start 64.936175 24.20327) (end 58.216175 17.48327) (width 0.2) (layer "F.Cu") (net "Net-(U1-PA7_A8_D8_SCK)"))
 (segment (start 38.286175 17.48327) (end 24.586175 31.18327) (width 0.2) (layer "F.Cu") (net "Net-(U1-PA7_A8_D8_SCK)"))
 (segment (start 58.216175 17.48327) (end 38.286175 17.48327) (width 0.2) (layer "F.Cu") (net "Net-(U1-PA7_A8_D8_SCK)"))
 (via (at 24.586175 31.18327) (size 0.6) (drill 0.3) (layers "F.Cu" "B.Cu") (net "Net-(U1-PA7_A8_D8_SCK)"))
 (segment (start 74.154653 17.08327) (end 36.146175 17.08327) (width 0.2) (layer "F.Cu") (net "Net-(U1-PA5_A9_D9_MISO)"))
 (segment (start 80.736175 23.664792) (end 74.154653 17.08327) (width 0.2) (layer "F.Cu") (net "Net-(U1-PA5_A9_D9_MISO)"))
 (segment (start 79.436175 29.20327) (end 80.736175 27.90327) (width 0.2) (layer "F.Cu") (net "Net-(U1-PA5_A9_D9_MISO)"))
 (segment (start 36.146175 17.08327) (end 24.586175 28.64327) (width 0.2) (layer "F.Cu") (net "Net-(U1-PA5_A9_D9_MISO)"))
 (segment (start 80.736175 27.90327) (end 80.736175 23.664792) (width 0.2) (layer "F.Cu") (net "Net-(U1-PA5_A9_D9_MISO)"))
 (via (at 24.586175 28.64327) (size 0.6) (drill 0.3) (layers "F.Cu" "B.Cu") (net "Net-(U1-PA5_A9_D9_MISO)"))
 (segment (start 34.186175 25.88327) (end 41.586175 18.48327) (width 0.2) (layer "F.Cu") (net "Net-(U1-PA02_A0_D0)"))
 (segment (start 34.186175 42.20327) (end 34.186175 25.88327) (width 0.2) (layer "F.Cu") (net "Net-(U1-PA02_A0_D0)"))
 (via (at 41.586175 18.48327) (size 0.6) (drill 0.3) (layers "F.Cu" "B.Cu") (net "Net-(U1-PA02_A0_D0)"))
 (segment (start 40.986175 21.62327) (end 41.586175 21.02327) (width 0.2) (layer "F.Cu") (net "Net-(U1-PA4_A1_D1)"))
 (segment (start 43.586175 31.60327) (end 43.586175 26.411799) (width 0.2) (layer "F.Cu") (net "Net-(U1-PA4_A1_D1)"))
 (segment (start 40.986175 23.811799) (end 40.986175 21.62327) (width 0.2) (layer "F.Cu") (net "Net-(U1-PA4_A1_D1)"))
 (segment (start 43.586175 26.411799) (end 40.986175 23.811799) (width 0.2) (layer "F.Cu") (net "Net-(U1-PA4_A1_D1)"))
 (segment (start 54.186175 42.20327) (end 43.586175 31.60327) (width 0.2) (layer "F.Cu") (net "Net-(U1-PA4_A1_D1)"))
 (via (at 41.586175 21.02327) (size 0.6) (drill 0.3) (layers "F.Cu" "B.Cu") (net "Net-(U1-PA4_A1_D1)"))
 (segment (start 57.586175 42.20327) (end 45.136175 29.75327) (width 0.2) (layer "F.Cu") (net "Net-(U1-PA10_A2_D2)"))
 (segment (start 45.136175 27.11327) (end 41.586175 23.56327) (width 0.2) (layer "F.Cu") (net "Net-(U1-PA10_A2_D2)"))
 (segment (start 45.136175 29.75327) (end 45.136175 27.11327) (width 0.2) (layer "F.Cu") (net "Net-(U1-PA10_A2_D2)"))
 (segment (start 74.186175 42.20327) (end 57.586175 42.20327) (width 0.2) (layer "F.Cu") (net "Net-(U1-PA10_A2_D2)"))
 (via (at 41.586175 23.56327) (size 0.6) (drill 0.3) (layers "F.Cu" "B.Cu") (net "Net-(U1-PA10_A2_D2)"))
 (segment (start 64.936175 29.20327) (end 63.521962 29.20327) (width 0.2) (layer "F.Cu") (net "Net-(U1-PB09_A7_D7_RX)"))
 (segment (start 40.426175 17.88327) (end 24.586175 33.72327) (width 0.2) (layer "F.Cu") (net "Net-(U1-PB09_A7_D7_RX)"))
 (segment (start 55.836175 19.65327) (end 54.066175 17.88327) (width 0.2) (layer "F.Cu") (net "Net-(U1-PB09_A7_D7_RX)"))
 (segment (start 54.066175 17.88327) (end 40.426175 17.88327) (width 0.2) (layer "F.Cu") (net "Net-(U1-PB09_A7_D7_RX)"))
 (segment (start 55.836175 21.517483) (end 55.836175 19.65327) (width 0.2) (layer "F.Cu") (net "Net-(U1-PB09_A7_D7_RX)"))
 (segment (start 63.521962 29.20327) (end 55.836175 21.517483) (width 0.2) (layer "F.Cu") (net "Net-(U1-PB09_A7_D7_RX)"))
 (via (at 24.586175 33.72327) (size 0.6) (drill 0.3) (layers "F.Cu" "B.Cu") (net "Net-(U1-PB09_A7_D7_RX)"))
 (segment (start 41.586175 33.899868) (end 41.586175 33.72327) (width 0.2) (layer "F.Cu") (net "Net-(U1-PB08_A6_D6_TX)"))
 (via (at 41.586175 33.72327) (size 0.6) (drill 0.3) (layers "F.Cu" "B.Cu") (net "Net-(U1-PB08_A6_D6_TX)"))
 (segment (start 49.296175 44.223371) (end 41.076074 36.00327) (width 0.2) (layer "F.Cu") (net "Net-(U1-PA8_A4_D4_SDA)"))
 (segment (start 39.586175 35.20327) (end 39.586175 30.00327) (width 0.2) (layer "F.Cu") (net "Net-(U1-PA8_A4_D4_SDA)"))
 (segment (start 49.296175 57.31327) (end 49.296175 44.223371) (width 0.2) (layer "F.Cu") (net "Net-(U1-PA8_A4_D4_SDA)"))
 (segment (start 41.076074 36.00327) (end 40.386175 36.00327) (width 0.2) (layer "F.Cu") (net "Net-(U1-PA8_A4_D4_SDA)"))
 (segment (start 40.946175 28.64327) (end 41.586175 28.64327) (width 0.2) (layer "F.Cu") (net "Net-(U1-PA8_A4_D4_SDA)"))
 (segment (start 54.186175 62.20327) (end 49.296175 57.31327) (width 0.2) (layer "F.Cu") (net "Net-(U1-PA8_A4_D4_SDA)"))
 (segment (start 40.386175 36.00327) (end 39.586175 35.20327) (width 0.2) (layer "F.Cu") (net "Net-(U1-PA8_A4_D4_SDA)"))
 (segment (start 39.586175 30.00327) (end 40.946175 28.64327) (width 0.2) (layer "F.Cu") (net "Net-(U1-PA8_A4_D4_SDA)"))
 (via (at 41.586175 28.64327) (size 0.6) (drill 0.3) (layers "F.Cu" "B.Cu") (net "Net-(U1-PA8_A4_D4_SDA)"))
 (segment (start 34.186175 48.126214) (end 35.586175 46.726214) (width 0.2) (layer "F.Cu") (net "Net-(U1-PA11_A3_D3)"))
 (segment (start 35.586175 32.60327) (end 41.586175 26.60327) (width 0.2) (layer "F.Cu") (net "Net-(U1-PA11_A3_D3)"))
 (segment (start 41.586175 26.60327) (end 41.586175 26.10327) (width 0.2) (layer "F.Cu") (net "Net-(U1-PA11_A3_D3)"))
 (segment (start 34.186175 62.20327) (end 34.186175 48.126214) (width 0.2) (layer "F.Cu") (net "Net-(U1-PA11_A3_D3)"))
 (segment (start 35.586175 46.726214) (end 35.586175 32.60327) (width 0.2) (layer "F.Cu") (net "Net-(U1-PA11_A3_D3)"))
 (via (at 41.586175 26.10327) (size 0.6) (drill 0.3) (layers "F.Cu" "B.Cu") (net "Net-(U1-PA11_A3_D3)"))
 (segment (start 55.986175 44.00327) (end 53.386175 44.00327) (width 0.2) (layer "F.Cu") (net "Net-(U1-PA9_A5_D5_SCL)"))
 (segment (start 74.186175 62.20327) (end 55.986175 44.00327) (width 0.2) (layer "F.Cu") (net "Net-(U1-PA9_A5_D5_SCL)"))
 (segment (start 53.386175 44.00327) (end 41.586175 32.20327) (width 0.2) (layer "F.Cu") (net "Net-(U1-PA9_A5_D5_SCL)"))
 (segment (start 41.586175 32.20327) (end 41.586175 31.18327) (width 0.2) (layer "F.Cu") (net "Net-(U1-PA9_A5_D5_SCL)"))
 (via (at 41.586175 31.18327) (size 0.6) (drill 0.3) (layers "F.Cu" "B.Cu") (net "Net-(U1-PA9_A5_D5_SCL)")))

